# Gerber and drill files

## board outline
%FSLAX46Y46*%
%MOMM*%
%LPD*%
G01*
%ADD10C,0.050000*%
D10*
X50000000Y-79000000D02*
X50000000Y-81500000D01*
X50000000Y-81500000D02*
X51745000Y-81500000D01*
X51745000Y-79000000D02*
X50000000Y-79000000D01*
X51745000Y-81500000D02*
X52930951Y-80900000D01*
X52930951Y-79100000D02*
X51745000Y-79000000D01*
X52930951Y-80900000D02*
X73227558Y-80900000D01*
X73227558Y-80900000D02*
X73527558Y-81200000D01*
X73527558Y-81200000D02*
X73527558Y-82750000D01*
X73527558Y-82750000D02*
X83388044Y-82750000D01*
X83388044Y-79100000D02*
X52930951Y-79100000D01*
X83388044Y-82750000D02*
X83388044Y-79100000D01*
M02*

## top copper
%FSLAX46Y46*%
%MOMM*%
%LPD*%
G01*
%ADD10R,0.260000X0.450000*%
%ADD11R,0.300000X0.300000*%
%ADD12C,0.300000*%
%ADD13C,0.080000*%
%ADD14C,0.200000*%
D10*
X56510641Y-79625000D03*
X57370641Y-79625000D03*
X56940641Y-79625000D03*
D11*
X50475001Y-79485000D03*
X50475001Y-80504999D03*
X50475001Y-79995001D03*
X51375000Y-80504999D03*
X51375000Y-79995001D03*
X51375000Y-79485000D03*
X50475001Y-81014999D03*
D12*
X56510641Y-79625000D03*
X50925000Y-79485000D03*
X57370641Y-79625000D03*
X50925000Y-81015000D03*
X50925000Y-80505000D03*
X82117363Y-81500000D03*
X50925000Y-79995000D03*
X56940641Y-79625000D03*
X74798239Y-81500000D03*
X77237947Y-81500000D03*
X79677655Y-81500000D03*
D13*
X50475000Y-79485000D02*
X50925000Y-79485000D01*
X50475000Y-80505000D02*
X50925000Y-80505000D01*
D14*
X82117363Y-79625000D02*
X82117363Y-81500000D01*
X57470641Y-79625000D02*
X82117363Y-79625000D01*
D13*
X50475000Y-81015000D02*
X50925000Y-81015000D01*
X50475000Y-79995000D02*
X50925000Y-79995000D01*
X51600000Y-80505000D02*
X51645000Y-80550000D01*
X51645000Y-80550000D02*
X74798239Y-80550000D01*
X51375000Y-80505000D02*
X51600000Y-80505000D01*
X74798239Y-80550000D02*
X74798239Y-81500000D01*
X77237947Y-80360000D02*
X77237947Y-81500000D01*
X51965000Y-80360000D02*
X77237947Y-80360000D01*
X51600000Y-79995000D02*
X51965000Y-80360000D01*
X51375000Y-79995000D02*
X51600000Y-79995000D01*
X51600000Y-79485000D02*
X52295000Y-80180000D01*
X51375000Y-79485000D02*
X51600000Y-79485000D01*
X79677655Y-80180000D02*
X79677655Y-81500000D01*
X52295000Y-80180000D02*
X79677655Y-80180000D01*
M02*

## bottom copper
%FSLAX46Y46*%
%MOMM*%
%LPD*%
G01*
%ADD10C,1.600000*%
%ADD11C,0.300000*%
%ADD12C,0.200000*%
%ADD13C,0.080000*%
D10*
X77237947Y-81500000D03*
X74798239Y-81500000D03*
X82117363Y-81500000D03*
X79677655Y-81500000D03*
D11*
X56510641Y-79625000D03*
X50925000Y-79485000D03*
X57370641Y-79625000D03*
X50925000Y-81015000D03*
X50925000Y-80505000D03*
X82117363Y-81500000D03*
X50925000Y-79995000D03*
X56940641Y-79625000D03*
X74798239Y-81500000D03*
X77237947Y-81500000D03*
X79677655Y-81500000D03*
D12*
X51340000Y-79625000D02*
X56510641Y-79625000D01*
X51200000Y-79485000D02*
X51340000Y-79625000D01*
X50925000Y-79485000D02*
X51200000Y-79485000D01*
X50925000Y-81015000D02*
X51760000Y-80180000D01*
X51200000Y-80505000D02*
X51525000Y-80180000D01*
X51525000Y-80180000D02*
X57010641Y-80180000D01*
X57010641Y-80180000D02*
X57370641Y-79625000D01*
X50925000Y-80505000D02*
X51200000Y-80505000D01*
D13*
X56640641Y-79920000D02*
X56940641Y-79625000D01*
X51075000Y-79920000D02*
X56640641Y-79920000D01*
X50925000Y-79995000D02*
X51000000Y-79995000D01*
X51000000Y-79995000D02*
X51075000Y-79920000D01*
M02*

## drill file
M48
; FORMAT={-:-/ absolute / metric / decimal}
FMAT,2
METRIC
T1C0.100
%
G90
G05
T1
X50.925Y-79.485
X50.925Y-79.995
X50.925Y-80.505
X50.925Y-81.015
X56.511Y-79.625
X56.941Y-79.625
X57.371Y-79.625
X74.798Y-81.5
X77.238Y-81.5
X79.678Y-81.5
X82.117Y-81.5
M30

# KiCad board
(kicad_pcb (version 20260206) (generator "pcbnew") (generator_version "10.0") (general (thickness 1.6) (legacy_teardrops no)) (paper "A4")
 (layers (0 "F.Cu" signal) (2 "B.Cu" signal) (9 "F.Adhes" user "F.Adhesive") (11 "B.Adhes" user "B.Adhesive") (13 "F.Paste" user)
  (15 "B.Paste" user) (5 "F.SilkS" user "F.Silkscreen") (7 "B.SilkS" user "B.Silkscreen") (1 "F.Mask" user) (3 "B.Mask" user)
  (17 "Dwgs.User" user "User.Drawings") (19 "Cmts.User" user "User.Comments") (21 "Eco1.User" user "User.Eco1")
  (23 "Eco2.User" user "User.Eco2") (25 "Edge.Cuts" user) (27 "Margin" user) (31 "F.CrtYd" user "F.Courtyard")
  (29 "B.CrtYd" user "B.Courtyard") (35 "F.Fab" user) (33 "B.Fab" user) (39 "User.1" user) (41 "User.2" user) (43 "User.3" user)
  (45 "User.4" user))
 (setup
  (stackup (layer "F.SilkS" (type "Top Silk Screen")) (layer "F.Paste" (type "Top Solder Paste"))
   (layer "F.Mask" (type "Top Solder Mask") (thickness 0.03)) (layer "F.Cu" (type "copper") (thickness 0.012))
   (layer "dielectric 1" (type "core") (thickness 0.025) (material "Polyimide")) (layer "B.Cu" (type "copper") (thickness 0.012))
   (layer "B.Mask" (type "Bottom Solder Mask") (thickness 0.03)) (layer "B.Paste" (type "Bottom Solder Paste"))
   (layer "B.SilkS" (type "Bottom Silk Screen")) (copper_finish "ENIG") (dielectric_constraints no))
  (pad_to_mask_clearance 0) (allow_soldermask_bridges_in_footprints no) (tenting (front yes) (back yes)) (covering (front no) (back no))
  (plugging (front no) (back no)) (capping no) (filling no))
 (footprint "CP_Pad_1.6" (layer "F.Cu") (at 82.117363 81.5)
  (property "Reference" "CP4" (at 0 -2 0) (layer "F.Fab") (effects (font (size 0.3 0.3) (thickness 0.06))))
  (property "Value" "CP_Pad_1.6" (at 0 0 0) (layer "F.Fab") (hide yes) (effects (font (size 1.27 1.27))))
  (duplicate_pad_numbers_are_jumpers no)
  (pad "1" smd circle (at 0 0) (size 1.6 1.6) (layers "B.Cu" "B.Mask") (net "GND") (solder_mask_margin 0.1)))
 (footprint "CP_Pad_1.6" (layer "F.Cu") (at 77.237947 81.5)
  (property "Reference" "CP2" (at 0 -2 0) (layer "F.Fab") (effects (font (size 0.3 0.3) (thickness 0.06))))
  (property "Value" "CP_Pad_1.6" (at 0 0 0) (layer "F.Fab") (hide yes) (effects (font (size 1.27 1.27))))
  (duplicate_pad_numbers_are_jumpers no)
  (pad "1" smd circle (at 0 0) (size 1.6 1.6) (layers "B.Cu" "B.Mask") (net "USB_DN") (solder_mask_margin 0.1)))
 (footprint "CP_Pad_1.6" (layer "F.Cu") (at 79.677655 81.5)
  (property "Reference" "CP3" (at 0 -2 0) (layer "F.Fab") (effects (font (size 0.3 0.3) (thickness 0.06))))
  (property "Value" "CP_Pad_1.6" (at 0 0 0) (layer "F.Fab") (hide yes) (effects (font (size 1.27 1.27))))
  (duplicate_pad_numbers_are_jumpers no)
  (pad "1" smd circle (at 0 0) (size 1.6 1.6) (layers "B.Cu" "B.Mask") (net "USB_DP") (solder_mask_margin 0.1)))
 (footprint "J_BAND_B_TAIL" (layer "F.Cu") (at 50.9 80.25)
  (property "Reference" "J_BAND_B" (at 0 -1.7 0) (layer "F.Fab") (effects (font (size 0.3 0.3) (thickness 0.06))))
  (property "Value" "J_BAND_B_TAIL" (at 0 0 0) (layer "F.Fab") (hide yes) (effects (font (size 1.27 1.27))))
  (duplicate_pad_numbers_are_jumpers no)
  (pad "1" smd rect (at -0.424999 -0.765) (size 0.3 0.3) (layers "F.Cu" "F.Mask") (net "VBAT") (solder_mask_margin 0.05)
   (thermal_bridge_angle 45))
  (pad "2" smd rect (at -0.424999 0.254999) (size 0.3 0.3) (layers "F.Cu" "F.Mask") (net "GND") (solder_mask_margin 0.05)
   (thermal_bridge_angle 45))
  (pad "3" smd rect (at -0.424999 -0.254999) (size 0.3 0.3) (layers "F.Cu" "F.Mask") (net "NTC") (solder_mask_margin 0.05)
   (thermal_bridge_angle 45))
  (pad "4" smd rect (at 0.475 0.254999) (size 0.3 0.3) (layers "F.Cu" "F.Mask") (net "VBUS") (solder_mask_margin 0.05)
   (thermal_bridge_angle 45))
  (pad "5" smd rect (at 0.475 -0.254999) (size 0.3 0.3) (layers "F.Cu" "F.Mask") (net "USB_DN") (solder_mask_margin 0.05)
   (thermal_bridge_angle 45))
  (pad "6" smd rect (at 0.475 -0.765) (size 0.3 0.3) (layers "F.Cu" "F.Mask") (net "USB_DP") (solder_mask_margin 0.05)
   (thermal_bridge_angle 45))
  (pad "7" smd rect (at -0.424999 0.764999) (size 0.3 0.3) (layers "F.Cu" "F.Mask") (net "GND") (solder_mask_margin 0.05)
   (thermal_bridge_angle 45)))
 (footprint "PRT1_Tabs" (layer "F.Cu") (at 56.940641 79.625)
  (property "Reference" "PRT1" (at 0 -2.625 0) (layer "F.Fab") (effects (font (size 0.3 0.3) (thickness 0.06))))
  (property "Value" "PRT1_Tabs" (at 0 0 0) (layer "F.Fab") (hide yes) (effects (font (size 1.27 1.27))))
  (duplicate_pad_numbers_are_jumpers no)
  (pad "1" smd rect (at -0.43 0) (size 0.26 0.45) (layers "F.Cu" "F.Mask") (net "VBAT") (solder_mask_margin 0.05) (thermal_bridge_angle 45))
  (pad "2" smd rect (at 0.43 0) (size 0.26 0.45) (layers "F.Cu" "F.Mask") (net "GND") (solder_mask_margin 0.05) (thermal_bridge_angle 45))
  (pad "3" smd rect (at 0 0) (size 0.26 0.45) (layers "F.Cu" "F.Mask") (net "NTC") (solder_mask_margin 0.05) (thermal_bridge_angle 45)))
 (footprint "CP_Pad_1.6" (layer "F.Cu") (at 74.798239 81.5)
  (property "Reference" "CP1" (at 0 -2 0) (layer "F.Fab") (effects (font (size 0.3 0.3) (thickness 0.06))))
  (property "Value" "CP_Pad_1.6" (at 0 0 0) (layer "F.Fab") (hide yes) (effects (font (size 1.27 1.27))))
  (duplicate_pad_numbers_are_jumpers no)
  (pad "1" smd circle (at 0 0) (size 1.6 1.6) (layers "B.Cu" "B.Mask") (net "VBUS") (solder_mask_margin 0.1)))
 (gr_line (start 50 79) (end 50 81.5) (stroke (width 0.05) (type default)) (layer "Edge.Cuts"))
 (gr_line (start 50 81.5) (end 51.745 81.5) (stroke (width 0.05) (type default)) (layer "Edge.Cuts"))
 (gr_line (start 51.745 79) (end 50 79) (stroke (width 0.05) (type default)) (layer "Edge.Cuts"))
 (gr_line (start 51.745 81.5) (end 52.930951 80.9) (stroke (width 0.05) (type default)) (layer "Edge.Cuts"))
 (gr_line (start 52.930951 79.1) (end 51.745 79) (stroke (width 0.05) (type default)) (layer "Edge.Cuts"))
 (gr_line (start 52.930951 80.9) (end 73.227558 80.9) (stroke (width 0.05) (type default)) (layer "Edge.Cuts"))
 (gr_line (start 73.227558 80.9) (end 73.527558 81.2) (stroke (width 0.05) (type default)) (layer "Edge.Cuts"))
 (gr_line (start 73.527558 81.2) (end 73.527558 82.75) (stroke (width 0.05) (type default)) (layer "Edge.Cuts"))
 (gr_line (start 73.527558 82.75) (end 83.388044 82.75) (stroke (width 0.05) (type default)) (layer "Edge.Cuts"))
 (gr_line (start 83.388044 79.1) (end 52.930951 79.1) (stroke (width 0.05) (type default)) (layer "Edge.Cuts"))
 (gr_line (start 83.388044 82.75) (end 83.388044 79.1) (stroke (width 0.05) (type default)) (layer "Edge.Cuts"))
 (segment (start 50.475 79.485) (end 50.925 79.485) (width 0.08) (layer "F.Cu") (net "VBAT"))
 (via (at 50.925 79.485) (size 0.3) (drill 0.1) (layers "F.Cu" "B.Cu") (tenting (front yes) (back yes)) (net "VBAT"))
 (via (at 56.510641 79.625) (size 0.3) (drill 0.1) (layers "F.Cu" "B.Cu") (tenting (front yes) (back yes)) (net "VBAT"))
 (segment (start 50.925 79.485) (end 51.2 79.485) (width 0.2) (layer "B.Cu") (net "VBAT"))
 (segment (start 51.34 79.625) (end 56.510641 79.625) (width 0.2) (layer "B.Cu") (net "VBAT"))
 (segment (start 51.2 79.485) (end 51.34 79.625) (width 0.2) (layer "B.Cu") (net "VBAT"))
 (segment (start 57.470641 79.625) (end 82.117363 79.625) (width 0.2) (layer "F.Cu") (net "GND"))
 (segment (start 50.475 81.015) (end 50.925 81.015) (width 0.08) (layer "F.Cu") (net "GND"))
 (segment (start 82.117363 79.625) (end 82.117363 81.5) (width 0.2) (layer "F.Cu") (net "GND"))
 (segment (start 50.475 80.505) (end 50.925 80.505) (width 0.08) (layer "F.Cu") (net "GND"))
 (via (at 50.925 81.015) (size 0.3) (drill 0.1) (layers "F.Cu" "B.Cu") (tenting (front yes) (back yes)) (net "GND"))
 (via (at 50.925 80.505) (size 0.3) (drill 0.1) (layers "F.Cu" "B.Cu") (tenting (front yes) (back yes)) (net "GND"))
 (via (at 82.117363 81.5) (size 0.3) (drill 0.1) (layers "F.Cu" "B.Cu") (tenting (front yes) (back yes)) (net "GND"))
 (via (at 57.370641 79.625) (size 0.3) (drill 0.1) (layers "F.Cu" "B.Cu") (tenting (front yes) (back yes)) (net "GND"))
 (segment (start 50.925 81.015) (end 51.76 80.18) (width 0.2) (layer "B.Cu") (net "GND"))
 (segment (start 50.925 80.505) (end 51.2 80.505) (width 0.2) (layer "B.Cu") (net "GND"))
 (segment (start 51.2 80.505) (end 51.525 80.18) (width 0.2) (layer "B.Cu") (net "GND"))
 (segment (start 57.010641 80.18) (end 57.370641 79.625) (width 0.2) (layer "B.Cu") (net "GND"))
 (segment (start 51.525 80.18) (end 57.010641 80.18) (width 0.2) (layer "B.Cu") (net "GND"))
 (segment (start 50.475 79.995) (end 50.925 79.995) (width 0.08) (layer "F.Cu") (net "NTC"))
 (via (at 50.925 79.995) (size 0.3) (drill 0.1) (layers "F.Cu" "B.Cu") (tenting (front yes) (back yes)) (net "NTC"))
 (via (at 56.940641 79.625) (size 0.3) (drill 0.1) (layers "F.Cu" "B.Cu") (tenting (front yes) (back yes)) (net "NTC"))
 (segment (start 51.075 79.92) (end 56.640641 79.92) (width 0.08) (layer "B.Cu") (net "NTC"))
 (segment (start 56.640641 79.92) (end 56.940641 79.625) (width 0.08) (layer "B.Cu") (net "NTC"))
 (segment (start 50.925 79.995) (end 51 79.995) (width 0.08) (layer "B.Cu") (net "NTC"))
 (segment (start 51 79.995) (end 51.075 79.92) (width 0.08) (layer "B.Cu") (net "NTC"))
 (segment (start 51.645 80.55) (end 74.798239 80.55) (width 0.08) (layer "F.Cu") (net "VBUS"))
 (segment (start 51.6 80.505) (end 51.645 80.55) (width 0.08) (layer "F.Cu") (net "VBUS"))
 (segment (start 51.375 80.505) (end 51.6 80.505) (width 0.08) (layer "F.Cu") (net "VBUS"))
 (segment (start 74.798239 80.55) (end 74.798239 81.5) (width 0.08) (layer "F.Cu") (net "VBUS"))
 (via (at 74.798239 81.5) (size 0.3) (drill 0.1) (layers "F.Cu" "B.Cu") (tenting (front yes) (back yes)) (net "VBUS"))
 (segment (start 51.6 79.995) (end 51.965 80.36) (width 0.08) (layer "F.Cu") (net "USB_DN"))
 (segment (start 51.375 79.995) (end 51.6 79.995) (width 0.08) (layer "F.Cu") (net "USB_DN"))
 (segment (start 77.237947 80.36) (end 77.237947 81.5) (width 0.08) (layer "F.Cu") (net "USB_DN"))
 (segment (start 51.965 80.36) (end 77.237947 80.36) (width 0.08) (layer "F.Cu") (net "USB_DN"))
 (via (at 77.237947 81.5) (size 0.3) (drill 0.1) (layers "F.Cu" "B.Cu") (tenting (front yes) (back yes)) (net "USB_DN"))
 (segment (start 51.6 79.485) (end 52.295 80.18) (width 0.08) (layer "F.Cu") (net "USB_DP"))
 (segment (start 79.677655 80.18) (end 79.677655 81.5) (width 0.08) (layer "F.Cu") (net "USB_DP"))
 (segment (start 51.375 79.485) (end 51.6 79.485) (width 0.08) (layer "F.Cu") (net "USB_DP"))
 (segment (start 52.295 80.18) (end 79.677655 80.18) (width 0.08) (layer "F.Cu") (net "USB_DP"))
 (via (at 79.677655 81.5) (size 0.3) (drill 0.1) (layers "F.Cu" "B.Cu") (tenting (front yes) (back yes)) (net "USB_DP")))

